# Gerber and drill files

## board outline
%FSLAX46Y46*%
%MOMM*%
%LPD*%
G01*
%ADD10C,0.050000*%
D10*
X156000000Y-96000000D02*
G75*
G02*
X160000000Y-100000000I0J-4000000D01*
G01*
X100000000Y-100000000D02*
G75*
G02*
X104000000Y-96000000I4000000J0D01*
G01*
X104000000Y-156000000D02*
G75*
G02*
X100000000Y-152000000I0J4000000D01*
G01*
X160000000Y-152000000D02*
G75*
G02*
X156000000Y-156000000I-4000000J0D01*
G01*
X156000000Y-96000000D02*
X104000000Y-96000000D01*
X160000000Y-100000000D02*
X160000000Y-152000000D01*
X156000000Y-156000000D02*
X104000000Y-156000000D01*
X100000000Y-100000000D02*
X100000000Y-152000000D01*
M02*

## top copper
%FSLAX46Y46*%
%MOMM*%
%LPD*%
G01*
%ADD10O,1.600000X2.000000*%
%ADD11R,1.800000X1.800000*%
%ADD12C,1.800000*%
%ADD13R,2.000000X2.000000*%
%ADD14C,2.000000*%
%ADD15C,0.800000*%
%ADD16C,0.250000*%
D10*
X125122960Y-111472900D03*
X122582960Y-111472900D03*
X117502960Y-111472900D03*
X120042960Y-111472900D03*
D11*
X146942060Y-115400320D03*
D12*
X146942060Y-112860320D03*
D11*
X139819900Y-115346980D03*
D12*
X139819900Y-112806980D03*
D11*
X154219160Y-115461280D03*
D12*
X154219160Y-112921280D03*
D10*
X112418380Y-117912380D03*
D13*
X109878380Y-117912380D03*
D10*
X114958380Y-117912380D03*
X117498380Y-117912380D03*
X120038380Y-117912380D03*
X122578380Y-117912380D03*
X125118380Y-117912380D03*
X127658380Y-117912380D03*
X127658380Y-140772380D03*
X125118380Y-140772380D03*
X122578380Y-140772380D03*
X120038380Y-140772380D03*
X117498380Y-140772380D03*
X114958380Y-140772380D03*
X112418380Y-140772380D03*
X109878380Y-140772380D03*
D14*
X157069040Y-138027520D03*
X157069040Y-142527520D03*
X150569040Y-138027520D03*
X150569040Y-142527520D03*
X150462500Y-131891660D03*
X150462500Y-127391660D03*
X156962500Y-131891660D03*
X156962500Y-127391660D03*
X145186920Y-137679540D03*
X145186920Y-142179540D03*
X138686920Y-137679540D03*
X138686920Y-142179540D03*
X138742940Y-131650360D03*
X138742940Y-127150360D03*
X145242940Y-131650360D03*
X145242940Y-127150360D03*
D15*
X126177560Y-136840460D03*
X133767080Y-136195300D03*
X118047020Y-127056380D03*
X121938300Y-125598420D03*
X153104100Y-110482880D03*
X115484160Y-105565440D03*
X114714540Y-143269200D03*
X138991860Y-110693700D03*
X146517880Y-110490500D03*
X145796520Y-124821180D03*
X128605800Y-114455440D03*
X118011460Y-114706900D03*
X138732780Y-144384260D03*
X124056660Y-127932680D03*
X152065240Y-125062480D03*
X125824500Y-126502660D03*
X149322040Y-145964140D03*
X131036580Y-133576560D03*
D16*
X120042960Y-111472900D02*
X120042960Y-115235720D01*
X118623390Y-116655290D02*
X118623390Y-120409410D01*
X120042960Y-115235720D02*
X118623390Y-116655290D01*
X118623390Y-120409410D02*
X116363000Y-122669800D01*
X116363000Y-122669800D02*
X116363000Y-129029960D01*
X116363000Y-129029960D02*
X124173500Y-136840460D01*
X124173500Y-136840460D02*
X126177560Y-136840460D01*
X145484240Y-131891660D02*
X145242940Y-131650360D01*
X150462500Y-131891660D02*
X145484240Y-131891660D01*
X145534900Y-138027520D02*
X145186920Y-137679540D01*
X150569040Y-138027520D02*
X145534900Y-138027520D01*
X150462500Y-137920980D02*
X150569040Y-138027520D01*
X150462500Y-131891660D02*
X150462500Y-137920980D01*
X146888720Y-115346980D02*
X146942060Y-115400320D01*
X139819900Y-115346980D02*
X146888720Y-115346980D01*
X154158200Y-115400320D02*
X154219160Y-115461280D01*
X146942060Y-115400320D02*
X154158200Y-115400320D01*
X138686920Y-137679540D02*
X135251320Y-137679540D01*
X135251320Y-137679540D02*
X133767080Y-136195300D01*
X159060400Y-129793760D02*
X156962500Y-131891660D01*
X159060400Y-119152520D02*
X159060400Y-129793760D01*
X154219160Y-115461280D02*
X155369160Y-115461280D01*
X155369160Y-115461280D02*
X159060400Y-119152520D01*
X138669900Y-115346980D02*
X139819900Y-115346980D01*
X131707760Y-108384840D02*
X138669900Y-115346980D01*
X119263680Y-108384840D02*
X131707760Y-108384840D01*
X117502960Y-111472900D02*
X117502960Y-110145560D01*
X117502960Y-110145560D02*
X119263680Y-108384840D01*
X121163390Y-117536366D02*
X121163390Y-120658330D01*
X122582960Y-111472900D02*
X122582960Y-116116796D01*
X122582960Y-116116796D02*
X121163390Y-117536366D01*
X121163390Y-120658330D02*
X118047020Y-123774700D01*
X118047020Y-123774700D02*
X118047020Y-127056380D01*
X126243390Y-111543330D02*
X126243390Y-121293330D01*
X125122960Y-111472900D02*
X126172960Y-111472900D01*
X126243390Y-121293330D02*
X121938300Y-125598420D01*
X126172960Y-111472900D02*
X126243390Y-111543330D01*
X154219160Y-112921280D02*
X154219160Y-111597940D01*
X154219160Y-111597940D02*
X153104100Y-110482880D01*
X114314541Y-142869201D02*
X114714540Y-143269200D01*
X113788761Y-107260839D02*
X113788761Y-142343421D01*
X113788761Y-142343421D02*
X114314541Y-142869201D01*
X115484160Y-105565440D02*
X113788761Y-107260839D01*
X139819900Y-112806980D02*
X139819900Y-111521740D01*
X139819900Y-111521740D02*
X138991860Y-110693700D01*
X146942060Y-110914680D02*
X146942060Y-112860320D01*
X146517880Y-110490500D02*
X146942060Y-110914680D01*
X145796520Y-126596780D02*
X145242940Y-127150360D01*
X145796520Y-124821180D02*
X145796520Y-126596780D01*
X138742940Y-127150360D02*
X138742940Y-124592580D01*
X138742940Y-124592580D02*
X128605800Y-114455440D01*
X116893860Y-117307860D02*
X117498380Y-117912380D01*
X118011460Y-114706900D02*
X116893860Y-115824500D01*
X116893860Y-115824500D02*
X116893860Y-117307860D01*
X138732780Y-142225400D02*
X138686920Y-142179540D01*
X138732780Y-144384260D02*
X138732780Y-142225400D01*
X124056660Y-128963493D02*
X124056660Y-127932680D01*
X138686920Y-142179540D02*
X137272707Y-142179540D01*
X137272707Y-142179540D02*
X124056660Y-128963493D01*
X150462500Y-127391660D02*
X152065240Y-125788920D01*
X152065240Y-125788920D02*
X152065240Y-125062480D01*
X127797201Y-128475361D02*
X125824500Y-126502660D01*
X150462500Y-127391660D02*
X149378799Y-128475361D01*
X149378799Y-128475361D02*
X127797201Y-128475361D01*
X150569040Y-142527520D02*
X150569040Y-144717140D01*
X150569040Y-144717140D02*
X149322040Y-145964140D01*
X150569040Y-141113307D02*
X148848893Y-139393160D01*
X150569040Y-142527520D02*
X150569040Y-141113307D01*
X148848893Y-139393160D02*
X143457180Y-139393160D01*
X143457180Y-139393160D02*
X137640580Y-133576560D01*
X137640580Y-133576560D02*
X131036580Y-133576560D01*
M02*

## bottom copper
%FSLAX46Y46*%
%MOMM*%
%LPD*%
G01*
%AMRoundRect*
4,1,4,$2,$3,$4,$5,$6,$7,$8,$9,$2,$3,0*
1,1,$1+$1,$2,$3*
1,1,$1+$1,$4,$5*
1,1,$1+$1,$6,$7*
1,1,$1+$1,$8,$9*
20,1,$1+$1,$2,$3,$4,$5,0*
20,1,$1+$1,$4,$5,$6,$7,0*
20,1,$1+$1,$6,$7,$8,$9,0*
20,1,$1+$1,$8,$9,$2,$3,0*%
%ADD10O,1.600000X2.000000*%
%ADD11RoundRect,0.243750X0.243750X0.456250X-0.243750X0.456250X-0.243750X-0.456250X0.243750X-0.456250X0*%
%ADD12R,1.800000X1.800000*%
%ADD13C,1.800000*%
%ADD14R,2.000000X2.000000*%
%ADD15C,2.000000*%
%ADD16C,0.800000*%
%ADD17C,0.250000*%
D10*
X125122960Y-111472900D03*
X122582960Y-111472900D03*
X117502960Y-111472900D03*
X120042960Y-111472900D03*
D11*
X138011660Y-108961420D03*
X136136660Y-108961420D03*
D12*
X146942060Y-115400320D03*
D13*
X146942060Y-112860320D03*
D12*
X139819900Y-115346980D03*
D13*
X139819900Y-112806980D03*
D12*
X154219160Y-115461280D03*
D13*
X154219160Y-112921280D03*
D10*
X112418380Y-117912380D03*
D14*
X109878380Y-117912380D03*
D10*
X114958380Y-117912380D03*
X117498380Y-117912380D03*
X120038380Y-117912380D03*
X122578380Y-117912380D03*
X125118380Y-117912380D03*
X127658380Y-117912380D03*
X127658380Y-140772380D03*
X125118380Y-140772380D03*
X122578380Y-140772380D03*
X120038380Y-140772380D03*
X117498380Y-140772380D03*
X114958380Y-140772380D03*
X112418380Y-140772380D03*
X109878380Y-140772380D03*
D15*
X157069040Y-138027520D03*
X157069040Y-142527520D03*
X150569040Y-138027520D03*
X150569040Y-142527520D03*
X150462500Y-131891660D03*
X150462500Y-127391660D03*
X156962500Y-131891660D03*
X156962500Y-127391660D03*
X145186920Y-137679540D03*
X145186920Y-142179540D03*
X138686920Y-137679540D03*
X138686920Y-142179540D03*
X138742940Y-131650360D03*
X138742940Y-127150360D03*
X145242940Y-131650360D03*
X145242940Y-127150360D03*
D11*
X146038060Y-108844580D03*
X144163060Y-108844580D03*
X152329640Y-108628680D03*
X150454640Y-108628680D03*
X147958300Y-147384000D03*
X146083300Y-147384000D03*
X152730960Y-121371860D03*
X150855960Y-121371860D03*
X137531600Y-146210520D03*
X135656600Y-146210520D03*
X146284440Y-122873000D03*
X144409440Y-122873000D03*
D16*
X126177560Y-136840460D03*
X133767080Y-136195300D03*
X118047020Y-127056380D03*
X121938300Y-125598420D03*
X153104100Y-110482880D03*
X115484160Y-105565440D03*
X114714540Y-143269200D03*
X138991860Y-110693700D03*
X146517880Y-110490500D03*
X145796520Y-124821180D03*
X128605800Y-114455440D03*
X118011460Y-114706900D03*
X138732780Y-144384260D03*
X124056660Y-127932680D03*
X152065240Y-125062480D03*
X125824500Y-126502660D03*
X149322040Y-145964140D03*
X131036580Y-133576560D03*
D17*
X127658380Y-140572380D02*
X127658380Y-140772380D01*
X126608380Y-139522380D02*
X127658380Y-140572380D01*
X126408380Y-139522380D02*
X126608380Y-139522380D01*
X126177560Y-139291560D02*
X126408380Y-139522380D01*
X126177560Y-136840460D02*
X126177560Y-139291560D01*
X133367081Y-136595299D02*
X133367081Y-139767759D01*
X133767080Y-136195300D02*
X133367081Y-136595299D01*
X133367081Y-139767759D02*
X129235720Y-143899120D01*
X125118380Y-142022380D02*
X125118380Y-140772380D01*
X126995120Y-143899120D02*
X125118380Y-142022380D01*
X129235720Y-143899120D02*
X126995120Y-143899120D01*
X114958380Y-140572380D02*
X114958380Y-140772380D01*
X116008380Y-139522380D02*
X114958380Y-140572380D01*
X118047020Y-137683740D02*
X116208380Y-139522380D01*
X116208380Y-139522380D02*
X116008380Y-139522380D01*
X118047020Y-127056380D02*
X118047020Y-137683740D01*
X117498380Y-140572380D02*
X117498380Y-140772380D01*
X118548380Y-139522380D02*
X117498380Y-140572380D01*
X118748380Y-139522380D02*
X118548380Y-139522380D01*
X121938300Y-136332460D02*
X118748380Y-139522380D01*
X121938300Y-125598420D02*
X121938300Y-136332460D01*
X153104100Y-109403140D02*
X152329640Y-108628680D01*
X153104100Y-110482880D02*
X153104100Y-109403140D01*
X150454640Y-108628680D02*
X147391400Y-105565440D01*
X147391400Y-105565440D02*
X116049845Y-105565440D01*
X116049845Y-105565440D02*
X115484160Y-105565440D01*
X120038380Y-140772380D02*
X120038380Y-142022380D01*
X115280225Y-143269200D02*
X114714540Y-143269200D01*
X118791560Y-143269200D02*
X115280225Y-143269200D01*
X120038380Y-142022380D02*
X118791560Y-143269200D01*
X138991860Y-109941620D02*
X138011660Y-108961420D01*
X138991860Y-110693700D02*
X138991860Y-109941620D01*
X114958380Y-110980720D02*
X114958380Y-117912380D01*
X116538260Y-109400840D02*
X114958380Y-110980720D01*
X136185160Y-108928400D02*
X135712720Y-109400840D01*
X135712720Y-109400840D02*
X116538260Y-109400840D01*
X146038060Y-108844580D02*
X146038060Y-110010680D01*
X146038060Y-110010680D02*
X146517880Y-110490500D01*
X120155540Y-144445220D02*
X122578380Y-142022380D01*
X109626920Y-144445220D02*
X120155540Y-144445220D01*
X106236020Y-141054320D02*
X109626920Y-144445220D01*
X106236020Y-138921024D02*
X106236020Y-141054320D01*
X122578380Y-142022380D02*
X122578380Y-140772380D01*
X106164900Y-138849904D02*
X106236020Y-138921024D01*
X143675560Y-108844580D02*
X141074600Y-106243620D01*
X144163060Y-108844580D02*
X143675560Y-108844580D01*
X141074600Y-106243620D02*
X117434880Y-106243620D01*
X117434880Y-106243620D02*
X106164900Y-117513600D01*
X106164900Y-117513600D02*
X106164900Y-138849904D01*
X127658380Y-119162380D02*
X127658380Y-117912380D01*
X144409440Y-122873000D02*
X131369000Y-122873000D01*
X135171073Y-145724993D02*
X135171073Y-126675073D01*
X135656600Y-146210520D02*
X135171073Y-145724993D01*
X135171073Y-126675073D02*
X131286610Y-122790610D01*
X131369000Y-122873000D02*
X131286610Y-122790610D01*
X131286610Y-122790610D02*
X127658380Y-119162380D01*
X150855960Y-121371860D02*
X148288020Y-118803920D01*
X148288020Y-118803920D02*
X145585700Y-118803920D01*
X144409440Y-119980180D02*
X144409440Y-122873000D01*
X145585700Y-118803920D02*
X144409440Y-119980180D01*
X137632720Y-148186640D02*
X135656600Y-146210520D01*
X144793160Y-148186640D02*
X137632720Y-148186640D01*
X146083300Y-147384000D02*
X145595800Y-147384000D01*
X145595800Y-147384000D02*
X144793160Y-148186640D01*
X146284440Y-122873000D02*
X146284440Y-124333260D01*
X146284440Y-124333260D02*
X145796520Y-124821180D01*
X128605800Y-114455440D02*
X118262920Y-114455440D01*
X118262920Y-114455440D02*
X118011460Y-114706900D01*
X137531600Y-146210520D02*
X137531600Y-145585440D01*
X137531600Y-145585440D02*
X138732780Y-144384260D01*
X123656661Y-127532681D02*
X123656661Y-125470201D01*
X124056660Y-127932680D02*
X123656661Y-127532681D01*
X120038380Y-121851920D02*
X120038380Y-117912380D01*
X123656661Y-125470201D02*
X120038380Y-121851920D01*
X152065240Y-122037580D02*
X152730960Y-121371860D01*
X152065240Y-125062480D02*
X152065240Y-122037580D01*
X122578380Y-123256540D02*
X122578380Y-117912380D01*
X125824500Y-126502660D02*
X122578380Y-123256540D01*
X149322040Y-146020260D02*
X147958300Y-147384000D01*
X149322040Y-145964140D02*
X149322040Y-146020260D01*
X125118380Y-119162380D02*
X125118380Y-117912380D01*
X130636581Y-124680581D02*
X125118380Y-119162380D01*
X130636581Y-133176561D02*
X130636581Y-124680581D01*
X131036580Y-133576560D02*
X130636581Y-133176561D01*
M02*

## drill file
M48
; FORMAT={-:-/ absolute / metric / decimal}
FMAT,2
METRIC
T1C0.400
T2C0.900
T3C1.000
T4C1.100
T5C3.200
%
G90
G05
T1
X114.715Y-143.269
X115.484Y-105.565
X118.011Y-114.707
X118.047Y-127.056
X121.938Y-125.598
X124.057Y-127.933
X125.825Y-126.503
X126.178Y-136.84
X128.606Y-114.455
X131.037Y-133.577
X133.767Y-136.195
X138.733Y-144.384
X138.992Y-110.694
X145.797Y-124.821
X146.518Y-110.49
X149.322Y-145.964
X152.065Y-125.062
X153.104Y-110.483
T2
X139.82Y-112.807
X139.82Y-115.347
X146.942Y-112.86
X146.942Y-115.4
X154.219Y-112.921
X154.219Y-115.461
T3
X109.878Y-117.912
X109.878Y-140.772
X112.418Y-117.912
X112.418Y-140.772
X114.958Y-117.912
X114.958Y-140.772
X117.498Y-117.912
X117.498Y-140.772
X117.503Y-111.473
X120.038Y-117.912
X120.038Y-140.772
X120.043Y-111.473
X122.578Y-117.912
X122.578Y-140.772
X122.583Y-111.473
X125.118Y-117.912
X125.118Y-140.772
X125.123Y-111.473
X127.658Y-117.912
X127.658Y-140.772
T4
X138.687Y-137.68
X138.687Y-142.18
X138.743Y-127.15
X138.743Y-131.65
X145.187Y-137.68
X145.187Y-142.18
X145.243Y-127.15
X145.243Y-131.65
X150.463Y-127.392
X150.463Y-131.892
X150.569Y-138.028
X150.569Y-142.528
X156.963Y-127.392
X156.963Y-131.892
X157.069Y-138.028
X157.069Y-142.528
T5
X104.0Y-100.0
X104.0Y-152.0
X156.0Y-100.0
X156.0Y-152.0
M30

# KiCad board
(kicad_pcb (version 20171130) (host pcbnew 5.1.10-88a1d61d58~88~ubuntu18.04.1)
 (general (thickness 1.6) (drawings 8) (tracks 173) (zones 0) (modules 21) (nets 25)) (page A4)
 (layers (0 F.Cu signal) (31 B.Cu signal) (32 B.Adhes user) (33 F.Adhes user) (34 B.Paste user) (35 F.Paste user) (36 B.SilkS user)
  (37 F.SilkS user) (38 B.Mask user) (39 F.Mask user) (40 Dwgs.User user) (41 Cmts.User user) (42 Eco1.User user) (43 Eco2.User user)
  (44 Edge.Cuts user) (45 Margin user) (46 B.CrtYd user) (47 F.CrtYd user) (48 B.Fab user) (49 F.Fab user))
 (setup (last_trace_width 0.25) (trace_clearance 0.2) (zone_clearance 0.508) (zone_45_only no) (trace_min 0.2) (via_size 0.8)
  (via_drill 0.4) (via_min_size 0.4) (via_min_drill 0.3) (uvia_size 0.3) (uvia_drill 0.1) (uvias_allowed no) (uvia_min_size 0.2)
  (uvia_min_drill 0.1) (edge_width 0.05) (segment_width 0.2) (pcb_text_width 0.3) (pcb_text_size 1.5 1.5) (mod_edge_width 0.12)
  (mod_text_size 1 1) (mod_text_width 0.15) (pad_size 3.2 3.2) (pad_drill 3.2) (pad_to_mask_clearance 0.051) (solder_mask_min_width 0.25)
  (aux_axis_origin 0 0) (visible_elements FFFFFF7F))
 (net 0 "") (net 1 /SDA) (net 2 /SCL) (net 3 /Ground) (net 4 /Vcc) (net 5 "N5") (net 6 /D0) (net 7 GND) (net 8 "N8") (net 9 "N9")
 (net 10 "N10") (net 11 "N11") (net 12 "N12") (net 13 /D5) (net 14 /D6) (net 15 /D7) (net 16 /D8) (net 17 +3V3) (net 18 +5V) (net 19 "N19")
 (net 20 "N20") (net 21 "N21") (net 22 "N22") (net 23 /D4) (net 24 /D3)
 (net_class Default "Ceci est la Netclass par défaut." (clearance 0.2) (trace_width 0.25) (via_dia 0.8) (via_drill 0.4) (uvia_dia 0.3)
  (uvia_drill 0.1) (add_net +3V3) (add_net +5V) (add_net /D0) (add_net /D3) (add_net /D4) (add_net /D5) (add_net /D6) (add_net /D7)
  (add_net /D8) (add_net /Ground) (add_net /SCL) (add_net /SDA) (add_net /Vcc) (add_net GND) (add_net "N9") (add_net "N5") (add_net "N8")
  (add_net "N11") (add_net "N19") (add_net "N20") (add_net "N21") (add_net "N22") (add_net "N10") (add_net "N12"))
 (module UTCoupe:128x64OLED (layer F.Cu) (at 121.12296 122.0729)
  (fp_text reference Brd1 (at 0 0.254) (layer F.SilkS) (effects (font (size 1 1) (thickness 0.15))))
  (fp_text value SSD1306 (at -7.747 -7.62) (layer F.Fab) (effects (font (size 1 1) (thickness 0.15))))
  (pad 4 thru_hole oval (at 4 -10.6 90) (size 2 1.6) (drill 1) (layers *.Cu *.Mask) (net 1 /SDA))
  (pad 3 thru_hole oval (at 1.46 -10.6 90) (size 2 1.6) (drill 1) (layers *.Cu *.Mask) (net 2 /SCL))
  (pad 1 thru_hole oval (at -3.62 -10.6 90) (size 2 1.6) (drill 1) (layers *.Cu *.Mask) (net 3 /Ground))
  (pad 2 thru_hole oval (at -1.08 -10.6 90) (size 2 1.6) (drill 1) (layers *.Cu *.Mask) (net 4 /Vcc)))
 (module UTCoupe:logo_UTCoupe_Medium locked (layer F.Cu) (at 124.7902 149.987)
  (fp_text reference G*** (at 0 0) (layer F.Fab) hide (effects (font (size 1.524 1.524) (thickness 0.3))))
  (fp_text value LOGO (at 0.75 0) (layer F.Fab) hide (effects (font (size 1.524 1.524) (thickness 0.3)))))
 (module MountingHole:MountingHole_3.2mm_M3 (layer F.Cu) (at 104 152 270)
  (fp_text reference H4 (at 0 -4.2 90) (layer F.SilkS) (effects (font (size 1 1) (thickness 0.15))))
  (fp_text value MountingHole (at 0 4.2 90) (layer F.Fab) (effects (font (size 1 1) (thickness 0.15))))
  (pad 1 np_thru_hole circle (at 0 0 270) (size 3.2 3.2) (drill 3.2) (layers *.Cu *.Mask)))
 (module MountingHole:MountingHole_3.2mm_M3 (layer F.Cu) (at 156 152 270)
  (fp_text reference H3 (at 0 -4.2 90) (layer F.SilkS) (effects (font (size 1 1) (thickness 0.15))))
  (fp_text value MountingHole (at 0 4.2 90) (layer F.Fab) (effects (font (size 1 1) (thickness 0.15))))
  (pad 1 np_thru_hole circle (at 0 0 270) (size 3.2 3.2) (drill 3.2) (layers *.Cu *.Mask)))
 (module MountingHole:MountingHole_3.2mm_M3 (layer F.Cu) (at 104 100 270)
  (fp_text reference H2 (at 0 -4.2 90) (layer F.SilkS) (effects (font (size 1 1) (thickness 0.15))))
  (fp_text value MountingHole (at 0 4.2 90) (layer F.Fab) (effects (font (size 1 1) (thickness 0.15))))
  (pad 1 np_thru_hole circle (at 0 0 270) (size 3.2 3.2) (drill 3.2) (layers *.Cu *.Mask)))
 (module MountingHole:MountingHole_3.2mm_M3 (layer F.Cu) (at 156 100 270)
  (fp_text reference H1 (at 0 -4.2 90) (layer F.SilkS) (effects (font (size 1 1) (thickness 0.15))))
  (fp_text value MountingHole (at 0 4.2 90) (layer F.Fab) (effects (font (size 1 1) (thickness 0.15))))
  (pad 1 np_thru_hole circle (at 0 0 270) (size 3.2 3.2) (drill 3.2) (layers *.Cu *.Mask)))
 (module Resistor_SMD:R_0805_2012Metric (layer B.Cu) (at 137.07416 108.96142 180)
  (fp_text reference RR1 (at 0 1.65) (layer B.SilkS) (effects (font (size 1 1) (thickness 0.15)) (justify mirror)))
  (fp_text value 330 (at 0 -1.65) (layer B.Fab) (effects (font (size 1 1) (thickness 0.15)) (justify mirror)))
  (pad 1 smd roundrect (at -0.9375 0 180) (size 0.975 1.4) (layers B.Cu B.Paste B.Mask) (roundrect_rratio 0.25) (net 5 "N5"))
  (pad 2 smd roundrect (at 0.9375 0 180) (size 0.975 1.4) (layers B.Cu B.Paste B.Mask) (roundrect_rratio 0.25) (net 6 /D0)))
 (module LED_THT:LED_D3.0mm (layer F.Cu) (at 146.94206 115.40032 90)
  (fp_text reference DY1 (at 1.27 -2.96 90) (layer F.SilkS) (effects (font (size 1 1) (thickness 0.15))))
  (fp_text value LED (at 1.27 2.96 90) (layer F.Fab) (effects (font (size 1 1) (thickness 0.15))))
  (pad 1 thru_hole rect (at 0 0 90) (size 1.8 1.8) (drill 0.9) (layers *.Cu *.Mask) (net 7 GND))
  (pad 2 thru_hole circle (at 2.54 0 90) (size 1.8 1.8) (drill 0.9) (layers *.Cu *.Mask) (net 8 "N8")))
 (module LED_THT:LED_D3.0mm (layer F.Cu) (at 139.8199 115.34698 90)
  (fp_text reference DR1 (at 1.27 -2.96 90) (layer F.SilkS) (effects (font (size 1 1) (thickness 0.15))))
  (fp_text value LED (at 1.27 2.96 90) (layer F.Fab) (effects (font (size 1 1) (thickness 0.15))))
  (pad 1 thru_hole rect (at 0 0 90) (size 1.8 1.8) (drill 0.9) (layers *.Cu *.Mask) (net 7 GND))
  (pad 2 thru_hole circle (at 2.54 0 90) (size 1.8 1.8) (drill 0.9) (layers *.Cu *.Mask) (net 5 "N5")))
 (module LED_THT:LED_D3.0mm (layer F.Cu) (at 154.21916 115.46128 90)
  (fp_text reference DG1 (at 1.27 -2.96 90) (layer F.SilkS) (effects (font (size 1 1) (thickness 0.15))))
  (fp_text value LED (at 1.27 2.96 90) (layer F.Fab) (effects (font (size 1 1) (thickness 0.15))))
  (pad 1 thru_hole rect (at 0 0 90) (size 1.8 1.8) (drill 0.9) (layers *.Cu *.Mask) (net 7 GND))
  (pad 2 thru_hole circle (at 2.54 0 90) (size 1.8 1.8) (drill 0.9) (layers *.Cu *.Mask) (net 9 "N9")))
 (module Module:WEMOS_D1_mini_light (layer B.Cu) (at 109.87838 117.91238 270)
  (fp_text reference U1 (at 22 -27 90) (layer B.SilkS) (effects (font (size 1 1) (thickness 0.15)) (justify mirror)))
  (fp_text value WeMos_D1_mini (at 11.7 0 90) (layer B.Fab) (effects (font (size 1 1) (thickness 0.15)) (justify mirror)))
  (pad 2 thru_hole oval (at 0 -2.54 270) (size 2 1.6) (drill 1) (layers *.Cu *.Mask) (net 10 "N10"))
  (pad 1 thru_hole rect (at 0 0 270) (size 2 2) (drill 1) (layers *.Cu *.Mask) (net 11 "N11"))
  (pad 3 thru_hole oval (at 0 -5.08 270) (size 2 1.6) (drill 1) (layers *.Cu *.Mask) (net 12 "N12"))
  (pad 4 thru_hole oval (at 0 -7.62 270) (size 2 1.6) (drill 1) (layers *.Cu *.Mask) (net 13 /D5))
  (pad 5 thru_hole oval (at 0 -10.16 270) (size 2 1.6) (drill 1) (layers *.Cu *.Mask) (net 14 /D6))
  (pad 6 thru_hole oval (at 0 -12.7 270) (size 2 1.6) (drill 1) (layers *.Cu *.Mask) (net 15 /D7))
  (pad 7 thru_hole oval (at 0 -15.24 270) (size 2 1.6) (drill 1) (layers *.Cu *.Mask) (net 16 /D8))
  (pad 8 thru_hole oval (at 0 -17.78 270) (size 2 1.6) (drill 1) (layers *.Cu *.Mask) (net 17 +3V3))
  (pad 9 thru_hole oval (at 22.86 -17.78 270) (size 2 1.6) (drill 1) (layers *.Cu *.Mask) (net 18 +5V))
  (pad 10 thru_hole oval (at 22.86 -15.24 270) (size 2 1.6) (drill 1) (layers *.Cu *.Mask) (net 7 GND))
  (pad 11 thru_hole oval (at 22.86 -12.7 270) (size 2 1.6) (drill 1) (layers *.Cu *.Mask) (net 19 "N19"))
  (pad 12 thru_hole oval (at 22.86 -10.16 270) (size 2 1.6) (drill 1) (layers *.Cu *.Mask) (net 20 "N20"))
  (pad 13 thru_hole oval (at 22.86 -7.62 270) (size 2 1.6) (drill 1) (layers *.Cu *.Mask) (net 1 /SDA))
  (pad 14 thru_hole oval (at 22.86 -5.08 270) (size 2 1.6) (drill 1) (layers *.Cu *.Mask) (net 2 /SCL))
  (pad 15 thru_hole oval (at 22.86 -2.54 270) (size 2 1.6) (drill 1) (layers *.Cu *.Mask) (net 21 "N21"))
  (pad 16 thru_hole oval (at 22.86 0 270) (size 2 1.6) (drill 1) (layers *.Cu *.Mask) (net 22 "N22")))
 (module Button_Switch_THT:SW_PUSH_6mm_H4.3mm (layer F.Cu) (at 157.06904 142.52752 180)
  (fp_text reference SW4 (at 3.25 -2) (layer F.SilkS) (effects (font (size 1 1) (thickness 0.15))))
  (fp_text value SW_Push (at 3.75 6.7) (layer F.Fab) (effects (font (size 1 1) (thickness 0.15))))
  (pad 2 thru_hole circle (at 0 4.5 270) (size 2 2) (drill 1.1) (layers *.Cu *.Mask) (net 7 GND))
  (pad 1 thru_hole circle (at 0 0 270) (size 2 2) (drill 1.1) (layers *.Cu *.Mask) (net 16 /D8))
  (pad 2 thru_hole circle (at 6.5 4.5 270) (size 2 2) (drill 1.1) (layers *.Cu *.Mask) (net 7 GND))
  (pad 1 thru_hole circle (at 6.5 0 270) (size 2 2) (drill 1.1) (layers *.Cu *.Mask) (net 16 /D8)))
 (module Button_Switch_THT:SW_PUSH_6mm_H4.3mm (layer F.Cu) (at 150.4625 127.39166)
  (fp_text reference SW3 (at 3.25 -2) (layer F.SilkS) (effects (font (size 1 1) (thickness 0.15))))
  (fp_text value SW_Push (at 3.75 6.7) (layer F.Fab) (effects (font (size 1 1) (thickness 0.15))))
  (pad 2 thru_hole circle (at 0 4.5 90) (size 2 2) (drill 1.1) (layers *.Cu *.Mask) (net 7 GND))
  (pad 1 thru_hole circle (at 0 0 90) (size 2 2) (drill 1.1) (layers *.Cu *.Mask) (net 15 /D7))
  (pad 2 thru_hole circle (at 6.5 4.5 90) (size 2 2) (drill 1.1) (layers *.Cu *.Mask) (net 7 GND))
  (pad 1 thru_hole circle (at 6.5 0 90) (size 2 2) (drill 1.1) (layers *.Cu *.Mask) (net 15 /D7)))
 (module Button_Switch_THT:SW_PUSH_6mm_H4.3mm (layer F.Cu) (at 145.18692 142.17954 180)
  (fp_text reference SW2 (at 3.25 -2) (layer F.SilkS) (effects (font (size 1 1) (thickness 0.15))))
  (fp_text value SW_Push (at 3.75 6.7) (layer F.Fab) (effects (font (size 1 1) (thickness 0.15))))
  (pad 2 thru_hole circle (at 0 4.5 270) (size 2 2) (drill 1.1) (layers *.Cu *.Mask) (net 7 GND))
  (pad 1 thru_hole circle (at 0 0 270) (size 2 2) (drill 1.1) (layers *.Cu *.Mask) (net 14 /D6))
  (pad 2 thru_hole circle (at 6.5 4.5 270) (size 2 2) (drill 1.1) (layers *.Cu *.Mask) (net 7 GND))
  (pad 1 thru_hole circle (at 6.5 0 270) (size 2 2) (drill 1.1) (layers *.Cu *.Mask) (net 14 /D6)))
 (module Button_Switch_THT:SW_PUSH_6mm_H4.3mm (layer F.Cu) (at 138.74294 127.15036)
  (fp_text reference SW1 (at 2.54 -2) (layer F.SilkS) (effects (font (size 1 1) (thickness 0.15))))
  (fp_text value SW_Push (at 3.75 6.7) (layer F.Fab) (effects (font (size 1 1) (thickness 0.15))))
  (pad 2 thru_hole circle (at 0 4.5 90) (size 2 2) (drill 1.1) (layers *.Cu *.Mask) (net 7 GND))
  (pad 1 thru_hole circle (at 0 0 90) (size 2 2) (drill 1.1) (layers *.Cu *.Mask) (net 13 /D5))
  (pad 2 thru_hole circle (at 6.5 4.5 90) (size 2 2) (drill 1.1) (layers *.Cu *.Mask) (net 7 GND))
  (pad 1 thru_hole circle (at 6.5 0 90) (size 2 2) (drill 1.1) (layers *.Cu *.Mask) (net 13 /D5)))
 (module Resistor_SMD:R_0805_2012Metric (layer B.Cu) (at 145.10056 108.84458 180)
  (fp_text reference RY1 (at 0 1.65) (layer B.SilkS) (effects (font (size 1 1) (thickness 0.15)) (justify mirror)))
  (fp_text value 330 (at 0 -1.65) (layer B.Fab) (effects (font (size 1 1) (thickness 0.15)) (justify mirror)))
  (pad 1 smd roundrect (at -0.9375 0 180) (size 0.975 1.4) (layers B.Cu B.Paste B.Mask) (roundrect_rratio 0.25) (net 8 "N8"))
  (pad 2 smd roundrect (at 0.9375 0 180) (size 0.975 1.4) (layers B.Cu B.Paste B.Mask) (roundrect_rratio 0.25) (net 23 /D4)))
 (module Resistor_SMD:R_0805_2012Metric (layer B.Cu) (at 151.39214 108.62868 180)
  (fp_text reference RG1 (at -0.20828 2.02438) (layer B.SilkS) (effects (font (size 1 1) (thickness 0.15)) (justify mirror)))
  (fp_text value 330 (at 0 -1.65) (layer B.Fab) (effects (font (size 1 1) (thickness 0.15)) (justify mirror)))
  (pad 1 smd roundrect (at -0.9375 0 180) (size 0.975 1.4) (layers B.Cu B.Paste B.Mask) (roundrect_rratio 0.25) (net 9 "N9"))
  (pad 2 smd roundrect (at 0.9375 0 180) (size 0.975 1.4) (layers B.Cu B.Paste B.Mask) (roundrect_rratio 0.25) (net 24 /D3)))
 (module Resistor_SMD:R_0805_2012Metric (layer B.Cu) (at 147.0208 147.384 180)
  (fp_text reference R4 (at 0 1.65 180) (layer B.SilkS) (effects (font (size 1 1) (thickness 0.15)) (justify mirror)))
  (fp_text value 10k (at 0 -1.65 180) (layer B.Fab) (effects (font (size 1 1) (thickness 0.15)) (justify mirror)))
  (pad 1 smd roundrect (at -0.9375 0 180) (size 0.975 1.4) (layers B.Cu B.Paste B.Mask) (roundrect_rratio 0.25) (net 16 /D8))
  (pad 2 smd roundrect (at 0.9375 0 180) (size 0.975 1.4) (layers B.Cu B.Paste B.Mask) (roundrect_rratio 0.25) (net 17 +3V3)))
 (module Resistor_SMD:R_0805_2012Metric (layer B.Cu) (at 151.79346 121.37186 180)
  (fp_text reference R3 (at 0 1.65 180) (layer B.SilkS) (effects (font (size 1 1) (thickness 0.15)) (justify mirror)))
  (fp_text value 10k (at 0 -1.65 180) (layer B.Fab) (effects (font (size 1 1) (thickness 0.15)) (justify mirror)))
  (pad 1 smd roundrect (at -0.9375 0 180) (size 0.975 1.4) (layers B.Cu B.Paste B.Mask) (roundrect_rratio 0.25) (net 15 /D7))
  (pad 2 smd roundrect (at 0.9375 0 180) (size 0.975 1.4) (layers B.Cu B.Paste B.Mask) (roundrect_rratio 0.25) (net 17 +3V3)))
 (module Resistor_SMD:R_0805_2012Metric (layer B.Cu) (at 136.5941 146.21052 180)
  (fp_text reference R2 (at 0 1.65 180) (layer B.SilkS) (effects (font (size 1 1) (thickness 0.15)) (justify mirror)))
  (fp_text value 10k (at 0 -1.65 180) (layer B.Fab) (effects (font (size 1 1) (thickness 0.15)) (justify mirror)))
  (pad 1 smd roundrect (at -0.9375 0 180) (size 0.975 1.4) (layers B.Cu B.Paste B.Mask) (roundrect_rratio 0.25) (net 14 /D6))
  (pad 2 smd roundrect (at 0.9375 0 180) (size 0.975 1.4) (layers B.Cu B.Paste B.Mask) (roundrect_rratio 0.25) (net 17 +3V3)))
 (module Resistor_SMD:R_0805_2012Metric (layer B.Cu) (at 145.34694 122.873 180)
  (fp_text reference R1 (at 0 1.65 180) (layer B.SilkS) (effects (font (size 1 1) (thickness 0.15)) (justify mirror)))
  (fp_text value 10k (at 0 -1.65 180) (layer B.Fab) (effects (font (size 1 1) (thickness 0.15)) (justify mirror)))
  (pad 1 smd roundrect (at -0.9375 0 180) (size 0.975 1.4) (layers B.Cu B.Paste B.Mask) (roundrect_rratio 0.25) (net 13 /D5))
  (pad 2 smd roundrect (at 0.9375 0 180) (size 0.975 1.4) (layers B.Cu B.Paste B.Mask) (roundrect_rratio 0.25) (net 17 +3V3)))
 (gr_arc (start 156 100) (end 160 100) (angle -90) (layer Edge.Cuts) (width 0.05))
 (gr_arc (start 104 100) (end 104 96) (angle -90) (layer Edge.Cuts) (width 0.05))
 (gr_arc (start 104 152) (end 104 156) (angle 90) (layer Edge.Cuts) (width 0.05))
 (gr_arc (start 156 152) (end 160 152) (angle 90) (layer Edge.Cuts) (width 0.05))
 (gr_line (start 156 96) (end 104 96) (layer Edge.Cuts) (width 0.05))
 (gr_line (start 160 100) (end 160 152) (layer Edge.Cuts) (width 0.05))
 (gr_line (start 156 156) (end 104 156) (layer Edge.Cuts) (width 0.05))
 (gr_line (start 100 100) (end 100 152) (layer Edge.Cuts) (width 0.05))
 (segment (start 120.04296 111.4729) (end 120.04296 115.23572) (width 0.25) (layer F.Cu) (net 4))
 (segment (start 118.62339 116.65529) (end 118.62339 120.40941) (width 0.25) (layer F.Cu) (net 4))
 (segment (start 120.04296 115.23572) (end 118.62339 116.65529) (width 0.25) (layer F.Cu) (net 4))
 (segment (start 118.62339 120.40941) (end 116.363 122.6698) (width 0.25) (layer F.Cu) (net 4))
 (segment (start 116.363 122.6698) (end 116.363 129.02996) (width 0.25) (layer F.Cu) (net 4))
 (via (at 126.17756 136.84046) (size 0.8) (drill 0.4) (layers F.Cu B.Cu) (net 4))
 (segment (start 116.363 129.02996) (end 124.1735 136.84046) (width 0.25) (layer F.Cu) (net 4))
 (segment (start 124.1735 136.84046) (end 126.17756 136.84046) (width 0.25) (layer F.Cu) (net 4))
 (segment (start 127.65838 140.57238) (end 127.65838 140.77238) (width 0.25) (layer B.Cu) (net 4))
 (segment (start 126.60838 139.52238) (end 127.65838 140.57238) (width 0.25) (layer B.Cu) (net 4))
 (segment (start 126.40838 139.52238) (end 126.60838 139.52238) (width 0.25) (layer B.Cu) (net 4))
 (segment (start 126.17756 139.29156) (end 126.40838 139.52238) (width 0.25) (layer B.Cu) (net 4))
 (segment (start 126.17756 136.84046) (end 126.17756 139.29156) (width 0.25) (layer B.Cu) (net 4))
 (segment (start 145.48424 131.89166) (end 145.24294 131.65036) (width 0.25) (layer F.Cu) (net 7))
 (segment (start 150.4625 131.89166) (end 145.48424 131.89166) (width 0.25) (layer F.Cu) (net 7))
 (segment (start 145.5349 138.02752) (end 145.18692 137.67954) (width 0.25) (layer F.Cu) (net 7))
 (segment (start 150.56904 138.02752) (end 145.5349 138.02752) (width 0.25) (layer F.Cu) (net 7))
 (segment (start 150.4625 137.92098) (end 150.56904 138.02752) (width 0.25) (layer F.Cu) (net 7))
 (segment (start 150.4625 131.89166) (end 150.4625 137.92098) (width 0.25) (layer F.Cu) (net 7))
 (segment (start 146.88872 115.34698) (end 146.94206 115.40032) (width 0.25) (layer F.Cu) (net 3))
 (segment (start 139.8199 115.34698) (end 146.88872 115.34698) (width 0.25) (layer F.Cu) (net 3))
 (segment (start 154.1582 115.40032) (end 154.21916 115.46128) (width 0.25) (layer F.Cu) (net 3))
 (segment (start 146.94206 115.40032) (end 154.1582 115.40032) (width 0.25) (layer F.Cu) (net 3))
 (via (at 133.76708 136.1953) (size 0.8) (drill 0.4) (layers F.Cu B.Cu) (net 7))
 (segment (start 138.68692 137.67954) (end 135.25132 137.67954) (width 0.25) (layer F.Cu) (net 7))
 (segment (start 135.25132 137.67954) (end 133.76708 136.1953) (width 0.25) (layer F.Cu) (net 7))
 (segment (start 133.367081 136.595299) (end 133.367081 139.767759) (width 0.25) (layer B.Cu) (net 7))
 (segment (start 133.76708 136.1953) (end 133.367081 136.595299) (width 0.25) (layer B.Cu) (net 7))
 (segment (start 133.367081 139.767759) (end 129.23572 143.89912) (width 0.25) (layer B.Cu) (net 7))
 (segment (start 125.11838 142.02238) (end 125.11838 140.77238) (width 0.25) (layer B.Cu) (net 7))
 (segment (start 126.99512 143.89912) (end 125.11838 142.02238) (width 0.25) (layer B.Cu) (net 7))
 (segment (start 129.23572 143.89912) (end 126.99512 143.89912) (width 0.25) (layer B.Cu) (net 7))
 (segment (start 159.0604 129.79376) (end 156.9625 131.89166) (width 0.25) (layer F.Cu) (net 3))
 (segment (start 159.0604 119.15252) (end 159.0604 129.79376) (width 0.25) (layer F.Cu) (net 3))
 (segment (start 154.21916 115.46128) (end 155.36916 115.46128) (width 0.25) (layer F.Cu) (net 3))
 (segment (start 155.36916 115.46128) (end 159.0604 119.15252) (width 0.25) (layer F.Cu) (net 3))
 (segment (start 138.6699 115.34698) (end 139.8199 115.34698) (width 0.25) (layer F.Cu) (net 3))
 (segment (start 131.70776 108.38484) (end 138.6699 115.34698) (width 0.25) (layer F.Cu) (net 3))
 (segment (start 119.26368 108.38484) (end 131.70776 108.38484) (width 0.25) (layer F.Cu) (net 3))
 (segment (start 117.50296 111.4729) (end 117.50296 110.14556) (width 0.25) (layer F.Cu) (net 3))
 (segment (start 117.50296 110.14556) (end 119.26368 108.38484) (width 0.25) (layer F.Cu) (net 3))
 (segment (start 121.16339 117.536366) (end 121.16339 120.65833) (width 0.25) (layer F.Cu) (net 2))
 (segment (start 122.58296 111.4729) (end 122.58296 116.116796) (width 0.25) (layer F.Cu) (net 2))
 (segment (start 122.58296 116.116796) (end 121.16339 117.536366) (width 0.25) (layer F.Cu) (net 2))
 (via (at 118.04702 127.05638) (size 0.8) (drill 0.4) (layers F.Cu B.Cu) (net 2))
 (segment (start 121.16339 120.65833) (end 118.04702 123.7747) (width 0.25) (layer F.Cu) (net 2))
 (segment (start 118.04702 123.7747) (end 118.04702 127.05638) (width 0.25) (layer F.Cu) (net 2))
 (segment (start 114.95838 140.57238) (end 114.95838 140.77238) (width 0.25) (layer B.Cu) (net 2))
 (segment (start 116.00838 139.52238) (end 114.95838 140.57238) (width 0.25) (layer B.Cu) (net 2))
 (segment (start 118.04702 137.68374) (end 116.20838 139.52238) (width 0.25) (layer B.Cu) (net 2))
 (segment (start 116.20838 139.52238) (end 116.00838 139.52238) (width 0.25) (layer B.Cu) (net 2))
 (segment (start 118.04702 127.05638) (end 118.04702 137.68374) (width 0.25) (layer B.Cu) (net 2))
 (via (at 121.9383 125.59842) (size 0.8) (drill 0.4) (layers F.Cu B.Cu) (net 1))
 (segment (start 126.24339 111.54333) (end 126.24339 121.29333) (width 0.25) (layer F.Cu) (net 1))
 (segment (start 125.12296 111.4729) (end 126.17296 111.4729) (width 0.25) (layer F.Cu) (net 1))
 (segment (start 126.24339 121.29333) (end 121.9383 125.59842) (width 0.25) (layer F.Cu) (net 1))
 (segment (start 126.17296 111.4729) (end 126.24339 111.54333) (width 0.25) (layer F.Cu) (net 1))
 (segment (start 117.49838 140.57238) (end 117.49838 140.77238) (width 0.25) (layer B.Cu) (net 1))
 (segment (start 118.54838 139.52238) (end 117.49838 140.57238) (width 0.25) (layer B.Cu) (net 1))
 (segment (start 118.74838 139.52238) (end 118.54838 139.52238) (width 0.25) (layer B.Cu) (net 1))
 (segment (start 121.9383 136.33246) (end 118.74838 139.52238) (width 0.25) (layer B.Cu) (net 1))
 (segment (start 121.9383 125.59842) (end 121.9383 136.33246) (width 0.25) (layer B.Cu) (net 1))
 (via (at 153.1041 110.48288) (size 0.8) (drill 0.4) (layers F.Cu B.Cu) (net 9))
 (segment (start 154.21916 112.92128) (end 154.21916 111.59794) (width 0.25) (layer F.Cu) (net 9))
 (segment (start 154.21916 111.59794) (end 153.1041 110.48288) (width 0.25) (layer F.Cu) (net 9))
 (segment (start 153.1041 109.40314) (end 152.32964 108.62868) (width 0.25) (layer B.Cu) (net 9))
 (segment (start 153.1041 110.48288) (end 153.1041 109.40314) (width 0.25) (layer B.Cu) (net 9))
 (via (at 115.48416 105.56544) (size 0.8) (drill 0.4) (layers F.Cu B.Cu) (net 24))
 (segment (start 150.45464 108.62868) (end 147.3914 105.56544) (width 0.25) (layer B.Cu) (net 24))
 (segment (start 147.3914 105.56544) (end 116.049845 105.56544) (width 0.25) (layer B.Cu) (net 24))
 (segment (start 116.049845 105.56544) (end 115.48416 105.56544) (width 0.25) (layer B.Cu) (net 24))
 (via (at 114.71454 143.2692) (size 0.8) (drill 0.4) (layers F.Cu B.Cu) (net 24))
 (segment (start 120.03838 140.77238) (end 120.03838 142.02238) (width 0.25) (layer B.Cu) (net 24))
 (segment (start 114.314541 142.869201) (end 114.71454 143.2692) (width 0.25) (layer F.Cu) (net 24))
 (segment (start 115.280225 143.2692) (end 114.71454 143.2692) (width 0.25) (layer B.Cu) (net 24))
 (segment (start 113.788761 107.260839) (end 113.788761 142.343421) (width 0.25) (layer F.Cu) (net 24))
 (segment (start 113.788761 142.343421) (end 114.314541 142.869201) (width 0.25) (layer F.Cu) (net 24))
 (segment (start 115.48416 105.56544) (end 113.788761 107.260839) (width 0.25) (layer F.Cu) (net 24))
 (segment (start 118.79156 143.2692) (end 115.280225 143.2692) (width 0.25) (layer B.Cu) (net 24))
 (segment (start 120.03838 142.02238) (end 118.79156 143.2692) (width 0.25) (layer B.Cu) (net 24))
 (via (at 138.99186 110.6937) (size 0.8) (drill 0.4) (layers F.Cu B.Cu) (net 5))
 (segment (start 139.8199 112.80698) (end 139.8199 111.52174) (width 0.25) (layer F.Cu) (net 5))
 (segment (start 139.8199 111.52174) (end 138.99186 110.6937) (width 0.25) (layer F.Cu) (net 5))
 (segment (start 138.99186 109.94162) (end 138.01166 108.96142) (width 0.25) (layer B.Cu) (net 5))
 (segment (start 138.99186 110.6937) (end 138.99186 109.94162) (width 0.25) (layer B.Cu) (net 5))
 (segment (start 114.95838 110.98072) (end 114.95838 117.91238) (width 0.25) (layer B.Cu) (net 6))
 (segment (start 116.53826 109.40084) (end 114.95838 110.98072) (width 0.25) (layer B.Cu) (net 6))
 (segment (start 136.18516 108.9284) (end 135.71272 109.40084) (width 0.25) (layer B.Cu) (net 6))
 (segment (start 135.71272 109.40084) (end 116.53826 109.40084) (width 0.25) (layer B.Cu) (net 6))
 (via (at 146.51788 110.4905) (size 0.8) (drill 0.4) (layers F.Cu B.Cu) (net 8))
 (segment (start 146.03806 108.84458) (end 146.03806 110.01068) (width 0.25) (layer B.Cu) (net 8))
 (segment (start 146.03806 110.01068) (end 146.51788 110.4905) (width 0.25) (layer B.Cu) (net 8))
 (segment (start 146.94206 110.91468) (end 146.94206 112.86032) (width 0.25) (layer F.Cu) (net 8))
 (segment (start 146.51788 110.4905) (end 146.94206 110.91468) (width 0.25) (layer F.Cu) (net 8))
 (segment (start 120.15554 144.44522) (end 122.57838 142.02238) (width 0.25) (layer B.Cu) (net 23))
 (segment (start 109.62692 144.44522) (end 120.15554 144.44522) (width 0.25) (layer B.Cu) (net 23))
 (segment (start 106.23602 141.05432) (end 109.62692 144.44522) (width 0.25) (layer B.Cu) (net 23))
 (segment (start 106.23602 138.921024) (end 106.23602 141.05432) (width 0.25) (layer B.Cu) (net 23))
 (segment (start 122.57838 142.02238) (end 122.57838 140.77238) (width 0.25) (layer B.Cu) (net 23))
 (segment (start 106.1649 138.849904) (end 106.23602 138.921024) (width 0.25) (layer B.Cu) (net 23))
 (segment (start 143.67556 108.84458) (end 141.0746 106.24362) (width 0.25) (layer B.Cu) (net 23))
 (segment (start 144.16306 108.84458) (end 143.67556 108.84458) (width 0.25) (layer B.Cu) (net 23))
 (segment (start 141.0746 106.24362) (end 117.43488 106.24362) (width 0.25) (layer B.Cu) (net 23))
 (segment (start 117.43488 106.24362) (end 106.1649 117.5136) (width 0.25) (layer B.Cu) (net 23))
 (segment (start 106.1649 117.5136) (end 106.1649 138.849904) (width 0.25) (layer B.Cu) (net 23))
 (segment (start 127.65838 119.16238) (end 127.65838 117.91238) (width 0.25) (layer B.Cu) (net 17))
 (segment (start 144.40944 122.873) (end 131.369 122.873) (width 0.25) (layer B.Cu) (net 17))
 (segment (start 135.171073 145.724993) (end 135.171073 126.675073) (width 0.25) (layer B.Cu) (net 17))
 (segment (start 135.6566 146.21052) (end 135.171073 145.724993) (width 0.25) (layer B.Cu) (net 17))
 (segment (start 135.171073 126.675073) (end 131.28661 122.79061) (width 0.25) (layer B.Cu) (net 17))
 (segment (start 131.369 122.873) (end 131.28661 122.79061) (width 0.25) (layer B.Cu) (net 17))
 (segment (start 131.28661 122.79061) (end 127.65838 119.16238) (width 0.25) (layer B.Cu) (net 17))
 (segment (start 150.85596 121.37186) (end 148.28802 118.80392) (width 0.25) (layer B.Cu) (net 17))
 (segment (start 148.28802 118.80392) (end 145.5857 118.80392) (width 0.25) (layer B.Cu) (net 17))
 (segment (start 144.40944 119.98018) (end 144.40944 122.873) (width 0.25) (layer B.Cu) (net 17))
 (segment (start 145.5857 118.80392) (end 144.40944 119.98018) (width 0.25) (layer B.Cu) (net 17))
 (segment (start 137.63272 148.18664) (end 135.6566 146.21052) (width 0.25) (layer B.Cu) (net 17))
 (segment (start 144.79316 148.18664) (end 137.63272 148.18664) (width 0.25) (layer B.Cu) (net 17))
 (segment (start 146.0833 147.384) (end 145.5958 147.384) (width 0.25) (layer B.Cu) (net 17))
 (segment (start 145.5958 147.384) (end 144.79316 148.18664) (width 0.25) (layer B.Cu) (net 17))
 (via (at 145.79652 124.82118) (size 0.8) (drill 0.4) (layers F.Cu B.Cu) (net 13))
 (segment (start 146.28444 122.873) (end 146.28444 124.33326) (width 0.25) (layer B.Cu) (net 13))
 (segment (start 146.28444 124.33326) (end 145.79652 124.82118) (width 0.25) (layer B.Cu) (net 13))
 (segment (start 145.79652 126.59678) (end 145.24294 127.15036) (width 0.25) (layer F.Cu) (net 13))
 (segment (start 145.79652 124.82118) (end 145.79652 126.59678) (width 0.25) (layer F.Cu) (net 13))
 (via (at 128.6058 114.45544) (size 0.8) (drill 0.4) (layers F.Cu B.Cu) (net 13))
 (segment (start 138.74294 127.15036) (end 138.74294 124.59258) (width 0.25) (layer F.Cu) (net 13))
 (segment (start 138.74294 124.59258) (end 128.6058 114.45544) (width 0.25) (layer F.Cu) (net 13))
 (via (at 118.01146 114.7069) (size 0.8) (drill 0.4) (layers F.Cu B.Cu) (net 13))
 (segment (start 128.6058 114.45544) (end 118.26292 114.45544) (width 0.25) (layer B.Cu) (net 13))
 (segment (start 118.26292 114.45544) (end 118.01146 114.7069) (width 0.25) (layer B.Cu) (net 13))
 (segment (start 116.89386 117.30786) (end 117.49838 117.91238) (width 0.25) (layer F.Cu) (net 13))
 (segment (start 118.01146 114.7069) (end 116.89386 115.8245) (width 0.25) (layer F.Cu) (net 13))
 (segment (start 116.89386 115.8245) (end 116.89386 117.30786) (width 0.25) (layer F.Cu) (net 13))
 (via (at 138.73278 144.38426) (size 0.8) (drill 0.4) (layers F.Cu B.Cu) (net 14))
 (segment (start 137.5316 146.21052) (end 137.5316 145.58544) (width 0.25) (layer B.Cu) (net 14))
 (segment (start 137.5316 145.58544) (end 138.73278 144.38426) (width 0.25) (layer B.Cu) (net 14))
 (segment (start 138.73278 142.2254) (end 138.68692 142.17954) (width 0.25) (layer F.Cu) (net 14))
 (segment (start 138.73278 144.38426) (end 138.73278 142.2254) (width 0.25) (layer F.Cu) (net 14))
 (via (at 124.05666 127.93268) (size 0.8) (drill 0.4) (layers F.Cu B.Cu) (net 14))
 (segment (start 124.05666 128.963493) (end 124.05666 127.93268) (width 0.25) (layer F.Cu) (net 14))
 (segment (start 138.68692 142.17954) (end 137.272707 142.17954) (width 0.25) (layer F.Cu) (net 14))
 (segment (start 137.272707 142.17954) (end 124.05666 128.963493) (width 0.25) (layer F.Cu) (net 14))
 (segment (start 123.656661 127.532681) (end 123.656661 125.470201) (width 0.25) (layer B.Cu) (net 14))
 (segment (start 124.05666 127.93268) (end 123.656661 127.532681) (width 0.25) (layer B.Cu) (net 14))
 (segment (start 120.03838 121.85192) (end 120.03838 117.91238) (width 0.25) (layer B.Cu) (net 14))
 (segment (start 123.656661 125.470201) (end 120.03838 121.85192) (width 0.25) (layer B.Cu) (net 14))
 (via (at 152.06524 125.06248) (size 0.8) (drill 0.4) (layers F.Cu B.Cu) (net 15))
 (segment (start 150.4625 127.39166) (end 152.06524 125.78892) (width 0.25) (layer F.Cu) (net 15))
 (segment (start 152.06524 125.78892) (end 152.06524 125.06248) (width 0.25) (layer F.Cu) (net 15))
 (segment (start 152.06524 122.03758) (end 152.73096 121.37186) (width 0.25) (layer B.Cu) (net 15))
 (segment (start 152.06524 125.06248) (end 152.06524 122.03758) (width 0.25) (layer B.Cu) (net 15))
 (via (at 125.8245 126.50266) (size 0.8) (drill 0.4) (layers F.Cu B.Cu) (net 15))
 (segment (start 127.797201 128.475361) (end 125.8245 126.50266) (width 0.25) (layer F.Cu) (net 15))
 (segment (start 150.4625 127.39166) (end 149.378799 128.475361) (width 0.25) (layer F.Cu) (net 15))
 (segment (start 149.378799 128.475361) (end 127.797201 128.475361) (width 0.25) (layer F.Cu) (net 15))
 (segment (start 122.57838 123.25654) (end 122.57838 117.91238) (width 0.25) (layer B.Cu) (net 15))
 (segment (start 125.8245 126.50266) (end 122.57838 123.25654) (width 0.25) (layer B.Cu) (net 15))
 (via (at 149.32204 145.96414) (size 0.8) (drill 0.4) (layers F.Cu B.Cu) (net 16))
 (segment (start 150.56904 142.52752) (end 150.56904 144.71714) (width 0.25) (layer F.Cu) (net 16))
 (segment (start 150.56904 144.71714) (end 149.32204 145.96414) (width 0.25) (layer F.Cu) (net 16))
 (segment (start 149.32204 146.02026) (end 147.9583 147.384) (width 0.25) (layer B.Cu) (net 16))
 (segment (start 149.32204 145.96414) (end 149.32204 146.02026) (width 0.25) (layer B.Cu) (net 16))
 (segment (start 150.56904 141.113307) (end 148.848893 139.39316) (width 0.25) (layer F.Cu) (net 16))
 (segment (start 150.56904 142.52752) (end 150.56904 141.113307) (width 0.25) (layer F.Cu) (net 16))
 (segment (start 148.848893 139.39316) (end 143.45718 139.39316) (width 0.25) (layer F.Cu) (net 16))
 (via (at 131.03658 133.57656) (size 0.8) (drill 0.4) (layers F.Cu B.Cu) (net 16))
 (segment (start 143.45718 139.39316) (end 137.64058 133.57656) (width 0.25) (layer F.Cu) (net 16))
 (segment (start 137.64058 133.57656) (end 131.03658 133.57656) (width 0.25) (layer F.Cu) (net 16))
 (segment (start 125.11838 119.16238) (end 125.11838 117.91238) (width 0.25) (layer B.Cu) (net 16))
 (segment (start 130.636581 124.680581) (end 125.11838 119.16238) (width 0.25) (layer B.Cu) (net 16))
 (segment (start 130.636581 133.176561) (end 130.636581 124.680581) (width 0.25) (layer B.Cu) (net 16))
 (segment (start 131.03658 133.57656) (end 130.636581 133.176561) (width 0.25) (layer B.Cu) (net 16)))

